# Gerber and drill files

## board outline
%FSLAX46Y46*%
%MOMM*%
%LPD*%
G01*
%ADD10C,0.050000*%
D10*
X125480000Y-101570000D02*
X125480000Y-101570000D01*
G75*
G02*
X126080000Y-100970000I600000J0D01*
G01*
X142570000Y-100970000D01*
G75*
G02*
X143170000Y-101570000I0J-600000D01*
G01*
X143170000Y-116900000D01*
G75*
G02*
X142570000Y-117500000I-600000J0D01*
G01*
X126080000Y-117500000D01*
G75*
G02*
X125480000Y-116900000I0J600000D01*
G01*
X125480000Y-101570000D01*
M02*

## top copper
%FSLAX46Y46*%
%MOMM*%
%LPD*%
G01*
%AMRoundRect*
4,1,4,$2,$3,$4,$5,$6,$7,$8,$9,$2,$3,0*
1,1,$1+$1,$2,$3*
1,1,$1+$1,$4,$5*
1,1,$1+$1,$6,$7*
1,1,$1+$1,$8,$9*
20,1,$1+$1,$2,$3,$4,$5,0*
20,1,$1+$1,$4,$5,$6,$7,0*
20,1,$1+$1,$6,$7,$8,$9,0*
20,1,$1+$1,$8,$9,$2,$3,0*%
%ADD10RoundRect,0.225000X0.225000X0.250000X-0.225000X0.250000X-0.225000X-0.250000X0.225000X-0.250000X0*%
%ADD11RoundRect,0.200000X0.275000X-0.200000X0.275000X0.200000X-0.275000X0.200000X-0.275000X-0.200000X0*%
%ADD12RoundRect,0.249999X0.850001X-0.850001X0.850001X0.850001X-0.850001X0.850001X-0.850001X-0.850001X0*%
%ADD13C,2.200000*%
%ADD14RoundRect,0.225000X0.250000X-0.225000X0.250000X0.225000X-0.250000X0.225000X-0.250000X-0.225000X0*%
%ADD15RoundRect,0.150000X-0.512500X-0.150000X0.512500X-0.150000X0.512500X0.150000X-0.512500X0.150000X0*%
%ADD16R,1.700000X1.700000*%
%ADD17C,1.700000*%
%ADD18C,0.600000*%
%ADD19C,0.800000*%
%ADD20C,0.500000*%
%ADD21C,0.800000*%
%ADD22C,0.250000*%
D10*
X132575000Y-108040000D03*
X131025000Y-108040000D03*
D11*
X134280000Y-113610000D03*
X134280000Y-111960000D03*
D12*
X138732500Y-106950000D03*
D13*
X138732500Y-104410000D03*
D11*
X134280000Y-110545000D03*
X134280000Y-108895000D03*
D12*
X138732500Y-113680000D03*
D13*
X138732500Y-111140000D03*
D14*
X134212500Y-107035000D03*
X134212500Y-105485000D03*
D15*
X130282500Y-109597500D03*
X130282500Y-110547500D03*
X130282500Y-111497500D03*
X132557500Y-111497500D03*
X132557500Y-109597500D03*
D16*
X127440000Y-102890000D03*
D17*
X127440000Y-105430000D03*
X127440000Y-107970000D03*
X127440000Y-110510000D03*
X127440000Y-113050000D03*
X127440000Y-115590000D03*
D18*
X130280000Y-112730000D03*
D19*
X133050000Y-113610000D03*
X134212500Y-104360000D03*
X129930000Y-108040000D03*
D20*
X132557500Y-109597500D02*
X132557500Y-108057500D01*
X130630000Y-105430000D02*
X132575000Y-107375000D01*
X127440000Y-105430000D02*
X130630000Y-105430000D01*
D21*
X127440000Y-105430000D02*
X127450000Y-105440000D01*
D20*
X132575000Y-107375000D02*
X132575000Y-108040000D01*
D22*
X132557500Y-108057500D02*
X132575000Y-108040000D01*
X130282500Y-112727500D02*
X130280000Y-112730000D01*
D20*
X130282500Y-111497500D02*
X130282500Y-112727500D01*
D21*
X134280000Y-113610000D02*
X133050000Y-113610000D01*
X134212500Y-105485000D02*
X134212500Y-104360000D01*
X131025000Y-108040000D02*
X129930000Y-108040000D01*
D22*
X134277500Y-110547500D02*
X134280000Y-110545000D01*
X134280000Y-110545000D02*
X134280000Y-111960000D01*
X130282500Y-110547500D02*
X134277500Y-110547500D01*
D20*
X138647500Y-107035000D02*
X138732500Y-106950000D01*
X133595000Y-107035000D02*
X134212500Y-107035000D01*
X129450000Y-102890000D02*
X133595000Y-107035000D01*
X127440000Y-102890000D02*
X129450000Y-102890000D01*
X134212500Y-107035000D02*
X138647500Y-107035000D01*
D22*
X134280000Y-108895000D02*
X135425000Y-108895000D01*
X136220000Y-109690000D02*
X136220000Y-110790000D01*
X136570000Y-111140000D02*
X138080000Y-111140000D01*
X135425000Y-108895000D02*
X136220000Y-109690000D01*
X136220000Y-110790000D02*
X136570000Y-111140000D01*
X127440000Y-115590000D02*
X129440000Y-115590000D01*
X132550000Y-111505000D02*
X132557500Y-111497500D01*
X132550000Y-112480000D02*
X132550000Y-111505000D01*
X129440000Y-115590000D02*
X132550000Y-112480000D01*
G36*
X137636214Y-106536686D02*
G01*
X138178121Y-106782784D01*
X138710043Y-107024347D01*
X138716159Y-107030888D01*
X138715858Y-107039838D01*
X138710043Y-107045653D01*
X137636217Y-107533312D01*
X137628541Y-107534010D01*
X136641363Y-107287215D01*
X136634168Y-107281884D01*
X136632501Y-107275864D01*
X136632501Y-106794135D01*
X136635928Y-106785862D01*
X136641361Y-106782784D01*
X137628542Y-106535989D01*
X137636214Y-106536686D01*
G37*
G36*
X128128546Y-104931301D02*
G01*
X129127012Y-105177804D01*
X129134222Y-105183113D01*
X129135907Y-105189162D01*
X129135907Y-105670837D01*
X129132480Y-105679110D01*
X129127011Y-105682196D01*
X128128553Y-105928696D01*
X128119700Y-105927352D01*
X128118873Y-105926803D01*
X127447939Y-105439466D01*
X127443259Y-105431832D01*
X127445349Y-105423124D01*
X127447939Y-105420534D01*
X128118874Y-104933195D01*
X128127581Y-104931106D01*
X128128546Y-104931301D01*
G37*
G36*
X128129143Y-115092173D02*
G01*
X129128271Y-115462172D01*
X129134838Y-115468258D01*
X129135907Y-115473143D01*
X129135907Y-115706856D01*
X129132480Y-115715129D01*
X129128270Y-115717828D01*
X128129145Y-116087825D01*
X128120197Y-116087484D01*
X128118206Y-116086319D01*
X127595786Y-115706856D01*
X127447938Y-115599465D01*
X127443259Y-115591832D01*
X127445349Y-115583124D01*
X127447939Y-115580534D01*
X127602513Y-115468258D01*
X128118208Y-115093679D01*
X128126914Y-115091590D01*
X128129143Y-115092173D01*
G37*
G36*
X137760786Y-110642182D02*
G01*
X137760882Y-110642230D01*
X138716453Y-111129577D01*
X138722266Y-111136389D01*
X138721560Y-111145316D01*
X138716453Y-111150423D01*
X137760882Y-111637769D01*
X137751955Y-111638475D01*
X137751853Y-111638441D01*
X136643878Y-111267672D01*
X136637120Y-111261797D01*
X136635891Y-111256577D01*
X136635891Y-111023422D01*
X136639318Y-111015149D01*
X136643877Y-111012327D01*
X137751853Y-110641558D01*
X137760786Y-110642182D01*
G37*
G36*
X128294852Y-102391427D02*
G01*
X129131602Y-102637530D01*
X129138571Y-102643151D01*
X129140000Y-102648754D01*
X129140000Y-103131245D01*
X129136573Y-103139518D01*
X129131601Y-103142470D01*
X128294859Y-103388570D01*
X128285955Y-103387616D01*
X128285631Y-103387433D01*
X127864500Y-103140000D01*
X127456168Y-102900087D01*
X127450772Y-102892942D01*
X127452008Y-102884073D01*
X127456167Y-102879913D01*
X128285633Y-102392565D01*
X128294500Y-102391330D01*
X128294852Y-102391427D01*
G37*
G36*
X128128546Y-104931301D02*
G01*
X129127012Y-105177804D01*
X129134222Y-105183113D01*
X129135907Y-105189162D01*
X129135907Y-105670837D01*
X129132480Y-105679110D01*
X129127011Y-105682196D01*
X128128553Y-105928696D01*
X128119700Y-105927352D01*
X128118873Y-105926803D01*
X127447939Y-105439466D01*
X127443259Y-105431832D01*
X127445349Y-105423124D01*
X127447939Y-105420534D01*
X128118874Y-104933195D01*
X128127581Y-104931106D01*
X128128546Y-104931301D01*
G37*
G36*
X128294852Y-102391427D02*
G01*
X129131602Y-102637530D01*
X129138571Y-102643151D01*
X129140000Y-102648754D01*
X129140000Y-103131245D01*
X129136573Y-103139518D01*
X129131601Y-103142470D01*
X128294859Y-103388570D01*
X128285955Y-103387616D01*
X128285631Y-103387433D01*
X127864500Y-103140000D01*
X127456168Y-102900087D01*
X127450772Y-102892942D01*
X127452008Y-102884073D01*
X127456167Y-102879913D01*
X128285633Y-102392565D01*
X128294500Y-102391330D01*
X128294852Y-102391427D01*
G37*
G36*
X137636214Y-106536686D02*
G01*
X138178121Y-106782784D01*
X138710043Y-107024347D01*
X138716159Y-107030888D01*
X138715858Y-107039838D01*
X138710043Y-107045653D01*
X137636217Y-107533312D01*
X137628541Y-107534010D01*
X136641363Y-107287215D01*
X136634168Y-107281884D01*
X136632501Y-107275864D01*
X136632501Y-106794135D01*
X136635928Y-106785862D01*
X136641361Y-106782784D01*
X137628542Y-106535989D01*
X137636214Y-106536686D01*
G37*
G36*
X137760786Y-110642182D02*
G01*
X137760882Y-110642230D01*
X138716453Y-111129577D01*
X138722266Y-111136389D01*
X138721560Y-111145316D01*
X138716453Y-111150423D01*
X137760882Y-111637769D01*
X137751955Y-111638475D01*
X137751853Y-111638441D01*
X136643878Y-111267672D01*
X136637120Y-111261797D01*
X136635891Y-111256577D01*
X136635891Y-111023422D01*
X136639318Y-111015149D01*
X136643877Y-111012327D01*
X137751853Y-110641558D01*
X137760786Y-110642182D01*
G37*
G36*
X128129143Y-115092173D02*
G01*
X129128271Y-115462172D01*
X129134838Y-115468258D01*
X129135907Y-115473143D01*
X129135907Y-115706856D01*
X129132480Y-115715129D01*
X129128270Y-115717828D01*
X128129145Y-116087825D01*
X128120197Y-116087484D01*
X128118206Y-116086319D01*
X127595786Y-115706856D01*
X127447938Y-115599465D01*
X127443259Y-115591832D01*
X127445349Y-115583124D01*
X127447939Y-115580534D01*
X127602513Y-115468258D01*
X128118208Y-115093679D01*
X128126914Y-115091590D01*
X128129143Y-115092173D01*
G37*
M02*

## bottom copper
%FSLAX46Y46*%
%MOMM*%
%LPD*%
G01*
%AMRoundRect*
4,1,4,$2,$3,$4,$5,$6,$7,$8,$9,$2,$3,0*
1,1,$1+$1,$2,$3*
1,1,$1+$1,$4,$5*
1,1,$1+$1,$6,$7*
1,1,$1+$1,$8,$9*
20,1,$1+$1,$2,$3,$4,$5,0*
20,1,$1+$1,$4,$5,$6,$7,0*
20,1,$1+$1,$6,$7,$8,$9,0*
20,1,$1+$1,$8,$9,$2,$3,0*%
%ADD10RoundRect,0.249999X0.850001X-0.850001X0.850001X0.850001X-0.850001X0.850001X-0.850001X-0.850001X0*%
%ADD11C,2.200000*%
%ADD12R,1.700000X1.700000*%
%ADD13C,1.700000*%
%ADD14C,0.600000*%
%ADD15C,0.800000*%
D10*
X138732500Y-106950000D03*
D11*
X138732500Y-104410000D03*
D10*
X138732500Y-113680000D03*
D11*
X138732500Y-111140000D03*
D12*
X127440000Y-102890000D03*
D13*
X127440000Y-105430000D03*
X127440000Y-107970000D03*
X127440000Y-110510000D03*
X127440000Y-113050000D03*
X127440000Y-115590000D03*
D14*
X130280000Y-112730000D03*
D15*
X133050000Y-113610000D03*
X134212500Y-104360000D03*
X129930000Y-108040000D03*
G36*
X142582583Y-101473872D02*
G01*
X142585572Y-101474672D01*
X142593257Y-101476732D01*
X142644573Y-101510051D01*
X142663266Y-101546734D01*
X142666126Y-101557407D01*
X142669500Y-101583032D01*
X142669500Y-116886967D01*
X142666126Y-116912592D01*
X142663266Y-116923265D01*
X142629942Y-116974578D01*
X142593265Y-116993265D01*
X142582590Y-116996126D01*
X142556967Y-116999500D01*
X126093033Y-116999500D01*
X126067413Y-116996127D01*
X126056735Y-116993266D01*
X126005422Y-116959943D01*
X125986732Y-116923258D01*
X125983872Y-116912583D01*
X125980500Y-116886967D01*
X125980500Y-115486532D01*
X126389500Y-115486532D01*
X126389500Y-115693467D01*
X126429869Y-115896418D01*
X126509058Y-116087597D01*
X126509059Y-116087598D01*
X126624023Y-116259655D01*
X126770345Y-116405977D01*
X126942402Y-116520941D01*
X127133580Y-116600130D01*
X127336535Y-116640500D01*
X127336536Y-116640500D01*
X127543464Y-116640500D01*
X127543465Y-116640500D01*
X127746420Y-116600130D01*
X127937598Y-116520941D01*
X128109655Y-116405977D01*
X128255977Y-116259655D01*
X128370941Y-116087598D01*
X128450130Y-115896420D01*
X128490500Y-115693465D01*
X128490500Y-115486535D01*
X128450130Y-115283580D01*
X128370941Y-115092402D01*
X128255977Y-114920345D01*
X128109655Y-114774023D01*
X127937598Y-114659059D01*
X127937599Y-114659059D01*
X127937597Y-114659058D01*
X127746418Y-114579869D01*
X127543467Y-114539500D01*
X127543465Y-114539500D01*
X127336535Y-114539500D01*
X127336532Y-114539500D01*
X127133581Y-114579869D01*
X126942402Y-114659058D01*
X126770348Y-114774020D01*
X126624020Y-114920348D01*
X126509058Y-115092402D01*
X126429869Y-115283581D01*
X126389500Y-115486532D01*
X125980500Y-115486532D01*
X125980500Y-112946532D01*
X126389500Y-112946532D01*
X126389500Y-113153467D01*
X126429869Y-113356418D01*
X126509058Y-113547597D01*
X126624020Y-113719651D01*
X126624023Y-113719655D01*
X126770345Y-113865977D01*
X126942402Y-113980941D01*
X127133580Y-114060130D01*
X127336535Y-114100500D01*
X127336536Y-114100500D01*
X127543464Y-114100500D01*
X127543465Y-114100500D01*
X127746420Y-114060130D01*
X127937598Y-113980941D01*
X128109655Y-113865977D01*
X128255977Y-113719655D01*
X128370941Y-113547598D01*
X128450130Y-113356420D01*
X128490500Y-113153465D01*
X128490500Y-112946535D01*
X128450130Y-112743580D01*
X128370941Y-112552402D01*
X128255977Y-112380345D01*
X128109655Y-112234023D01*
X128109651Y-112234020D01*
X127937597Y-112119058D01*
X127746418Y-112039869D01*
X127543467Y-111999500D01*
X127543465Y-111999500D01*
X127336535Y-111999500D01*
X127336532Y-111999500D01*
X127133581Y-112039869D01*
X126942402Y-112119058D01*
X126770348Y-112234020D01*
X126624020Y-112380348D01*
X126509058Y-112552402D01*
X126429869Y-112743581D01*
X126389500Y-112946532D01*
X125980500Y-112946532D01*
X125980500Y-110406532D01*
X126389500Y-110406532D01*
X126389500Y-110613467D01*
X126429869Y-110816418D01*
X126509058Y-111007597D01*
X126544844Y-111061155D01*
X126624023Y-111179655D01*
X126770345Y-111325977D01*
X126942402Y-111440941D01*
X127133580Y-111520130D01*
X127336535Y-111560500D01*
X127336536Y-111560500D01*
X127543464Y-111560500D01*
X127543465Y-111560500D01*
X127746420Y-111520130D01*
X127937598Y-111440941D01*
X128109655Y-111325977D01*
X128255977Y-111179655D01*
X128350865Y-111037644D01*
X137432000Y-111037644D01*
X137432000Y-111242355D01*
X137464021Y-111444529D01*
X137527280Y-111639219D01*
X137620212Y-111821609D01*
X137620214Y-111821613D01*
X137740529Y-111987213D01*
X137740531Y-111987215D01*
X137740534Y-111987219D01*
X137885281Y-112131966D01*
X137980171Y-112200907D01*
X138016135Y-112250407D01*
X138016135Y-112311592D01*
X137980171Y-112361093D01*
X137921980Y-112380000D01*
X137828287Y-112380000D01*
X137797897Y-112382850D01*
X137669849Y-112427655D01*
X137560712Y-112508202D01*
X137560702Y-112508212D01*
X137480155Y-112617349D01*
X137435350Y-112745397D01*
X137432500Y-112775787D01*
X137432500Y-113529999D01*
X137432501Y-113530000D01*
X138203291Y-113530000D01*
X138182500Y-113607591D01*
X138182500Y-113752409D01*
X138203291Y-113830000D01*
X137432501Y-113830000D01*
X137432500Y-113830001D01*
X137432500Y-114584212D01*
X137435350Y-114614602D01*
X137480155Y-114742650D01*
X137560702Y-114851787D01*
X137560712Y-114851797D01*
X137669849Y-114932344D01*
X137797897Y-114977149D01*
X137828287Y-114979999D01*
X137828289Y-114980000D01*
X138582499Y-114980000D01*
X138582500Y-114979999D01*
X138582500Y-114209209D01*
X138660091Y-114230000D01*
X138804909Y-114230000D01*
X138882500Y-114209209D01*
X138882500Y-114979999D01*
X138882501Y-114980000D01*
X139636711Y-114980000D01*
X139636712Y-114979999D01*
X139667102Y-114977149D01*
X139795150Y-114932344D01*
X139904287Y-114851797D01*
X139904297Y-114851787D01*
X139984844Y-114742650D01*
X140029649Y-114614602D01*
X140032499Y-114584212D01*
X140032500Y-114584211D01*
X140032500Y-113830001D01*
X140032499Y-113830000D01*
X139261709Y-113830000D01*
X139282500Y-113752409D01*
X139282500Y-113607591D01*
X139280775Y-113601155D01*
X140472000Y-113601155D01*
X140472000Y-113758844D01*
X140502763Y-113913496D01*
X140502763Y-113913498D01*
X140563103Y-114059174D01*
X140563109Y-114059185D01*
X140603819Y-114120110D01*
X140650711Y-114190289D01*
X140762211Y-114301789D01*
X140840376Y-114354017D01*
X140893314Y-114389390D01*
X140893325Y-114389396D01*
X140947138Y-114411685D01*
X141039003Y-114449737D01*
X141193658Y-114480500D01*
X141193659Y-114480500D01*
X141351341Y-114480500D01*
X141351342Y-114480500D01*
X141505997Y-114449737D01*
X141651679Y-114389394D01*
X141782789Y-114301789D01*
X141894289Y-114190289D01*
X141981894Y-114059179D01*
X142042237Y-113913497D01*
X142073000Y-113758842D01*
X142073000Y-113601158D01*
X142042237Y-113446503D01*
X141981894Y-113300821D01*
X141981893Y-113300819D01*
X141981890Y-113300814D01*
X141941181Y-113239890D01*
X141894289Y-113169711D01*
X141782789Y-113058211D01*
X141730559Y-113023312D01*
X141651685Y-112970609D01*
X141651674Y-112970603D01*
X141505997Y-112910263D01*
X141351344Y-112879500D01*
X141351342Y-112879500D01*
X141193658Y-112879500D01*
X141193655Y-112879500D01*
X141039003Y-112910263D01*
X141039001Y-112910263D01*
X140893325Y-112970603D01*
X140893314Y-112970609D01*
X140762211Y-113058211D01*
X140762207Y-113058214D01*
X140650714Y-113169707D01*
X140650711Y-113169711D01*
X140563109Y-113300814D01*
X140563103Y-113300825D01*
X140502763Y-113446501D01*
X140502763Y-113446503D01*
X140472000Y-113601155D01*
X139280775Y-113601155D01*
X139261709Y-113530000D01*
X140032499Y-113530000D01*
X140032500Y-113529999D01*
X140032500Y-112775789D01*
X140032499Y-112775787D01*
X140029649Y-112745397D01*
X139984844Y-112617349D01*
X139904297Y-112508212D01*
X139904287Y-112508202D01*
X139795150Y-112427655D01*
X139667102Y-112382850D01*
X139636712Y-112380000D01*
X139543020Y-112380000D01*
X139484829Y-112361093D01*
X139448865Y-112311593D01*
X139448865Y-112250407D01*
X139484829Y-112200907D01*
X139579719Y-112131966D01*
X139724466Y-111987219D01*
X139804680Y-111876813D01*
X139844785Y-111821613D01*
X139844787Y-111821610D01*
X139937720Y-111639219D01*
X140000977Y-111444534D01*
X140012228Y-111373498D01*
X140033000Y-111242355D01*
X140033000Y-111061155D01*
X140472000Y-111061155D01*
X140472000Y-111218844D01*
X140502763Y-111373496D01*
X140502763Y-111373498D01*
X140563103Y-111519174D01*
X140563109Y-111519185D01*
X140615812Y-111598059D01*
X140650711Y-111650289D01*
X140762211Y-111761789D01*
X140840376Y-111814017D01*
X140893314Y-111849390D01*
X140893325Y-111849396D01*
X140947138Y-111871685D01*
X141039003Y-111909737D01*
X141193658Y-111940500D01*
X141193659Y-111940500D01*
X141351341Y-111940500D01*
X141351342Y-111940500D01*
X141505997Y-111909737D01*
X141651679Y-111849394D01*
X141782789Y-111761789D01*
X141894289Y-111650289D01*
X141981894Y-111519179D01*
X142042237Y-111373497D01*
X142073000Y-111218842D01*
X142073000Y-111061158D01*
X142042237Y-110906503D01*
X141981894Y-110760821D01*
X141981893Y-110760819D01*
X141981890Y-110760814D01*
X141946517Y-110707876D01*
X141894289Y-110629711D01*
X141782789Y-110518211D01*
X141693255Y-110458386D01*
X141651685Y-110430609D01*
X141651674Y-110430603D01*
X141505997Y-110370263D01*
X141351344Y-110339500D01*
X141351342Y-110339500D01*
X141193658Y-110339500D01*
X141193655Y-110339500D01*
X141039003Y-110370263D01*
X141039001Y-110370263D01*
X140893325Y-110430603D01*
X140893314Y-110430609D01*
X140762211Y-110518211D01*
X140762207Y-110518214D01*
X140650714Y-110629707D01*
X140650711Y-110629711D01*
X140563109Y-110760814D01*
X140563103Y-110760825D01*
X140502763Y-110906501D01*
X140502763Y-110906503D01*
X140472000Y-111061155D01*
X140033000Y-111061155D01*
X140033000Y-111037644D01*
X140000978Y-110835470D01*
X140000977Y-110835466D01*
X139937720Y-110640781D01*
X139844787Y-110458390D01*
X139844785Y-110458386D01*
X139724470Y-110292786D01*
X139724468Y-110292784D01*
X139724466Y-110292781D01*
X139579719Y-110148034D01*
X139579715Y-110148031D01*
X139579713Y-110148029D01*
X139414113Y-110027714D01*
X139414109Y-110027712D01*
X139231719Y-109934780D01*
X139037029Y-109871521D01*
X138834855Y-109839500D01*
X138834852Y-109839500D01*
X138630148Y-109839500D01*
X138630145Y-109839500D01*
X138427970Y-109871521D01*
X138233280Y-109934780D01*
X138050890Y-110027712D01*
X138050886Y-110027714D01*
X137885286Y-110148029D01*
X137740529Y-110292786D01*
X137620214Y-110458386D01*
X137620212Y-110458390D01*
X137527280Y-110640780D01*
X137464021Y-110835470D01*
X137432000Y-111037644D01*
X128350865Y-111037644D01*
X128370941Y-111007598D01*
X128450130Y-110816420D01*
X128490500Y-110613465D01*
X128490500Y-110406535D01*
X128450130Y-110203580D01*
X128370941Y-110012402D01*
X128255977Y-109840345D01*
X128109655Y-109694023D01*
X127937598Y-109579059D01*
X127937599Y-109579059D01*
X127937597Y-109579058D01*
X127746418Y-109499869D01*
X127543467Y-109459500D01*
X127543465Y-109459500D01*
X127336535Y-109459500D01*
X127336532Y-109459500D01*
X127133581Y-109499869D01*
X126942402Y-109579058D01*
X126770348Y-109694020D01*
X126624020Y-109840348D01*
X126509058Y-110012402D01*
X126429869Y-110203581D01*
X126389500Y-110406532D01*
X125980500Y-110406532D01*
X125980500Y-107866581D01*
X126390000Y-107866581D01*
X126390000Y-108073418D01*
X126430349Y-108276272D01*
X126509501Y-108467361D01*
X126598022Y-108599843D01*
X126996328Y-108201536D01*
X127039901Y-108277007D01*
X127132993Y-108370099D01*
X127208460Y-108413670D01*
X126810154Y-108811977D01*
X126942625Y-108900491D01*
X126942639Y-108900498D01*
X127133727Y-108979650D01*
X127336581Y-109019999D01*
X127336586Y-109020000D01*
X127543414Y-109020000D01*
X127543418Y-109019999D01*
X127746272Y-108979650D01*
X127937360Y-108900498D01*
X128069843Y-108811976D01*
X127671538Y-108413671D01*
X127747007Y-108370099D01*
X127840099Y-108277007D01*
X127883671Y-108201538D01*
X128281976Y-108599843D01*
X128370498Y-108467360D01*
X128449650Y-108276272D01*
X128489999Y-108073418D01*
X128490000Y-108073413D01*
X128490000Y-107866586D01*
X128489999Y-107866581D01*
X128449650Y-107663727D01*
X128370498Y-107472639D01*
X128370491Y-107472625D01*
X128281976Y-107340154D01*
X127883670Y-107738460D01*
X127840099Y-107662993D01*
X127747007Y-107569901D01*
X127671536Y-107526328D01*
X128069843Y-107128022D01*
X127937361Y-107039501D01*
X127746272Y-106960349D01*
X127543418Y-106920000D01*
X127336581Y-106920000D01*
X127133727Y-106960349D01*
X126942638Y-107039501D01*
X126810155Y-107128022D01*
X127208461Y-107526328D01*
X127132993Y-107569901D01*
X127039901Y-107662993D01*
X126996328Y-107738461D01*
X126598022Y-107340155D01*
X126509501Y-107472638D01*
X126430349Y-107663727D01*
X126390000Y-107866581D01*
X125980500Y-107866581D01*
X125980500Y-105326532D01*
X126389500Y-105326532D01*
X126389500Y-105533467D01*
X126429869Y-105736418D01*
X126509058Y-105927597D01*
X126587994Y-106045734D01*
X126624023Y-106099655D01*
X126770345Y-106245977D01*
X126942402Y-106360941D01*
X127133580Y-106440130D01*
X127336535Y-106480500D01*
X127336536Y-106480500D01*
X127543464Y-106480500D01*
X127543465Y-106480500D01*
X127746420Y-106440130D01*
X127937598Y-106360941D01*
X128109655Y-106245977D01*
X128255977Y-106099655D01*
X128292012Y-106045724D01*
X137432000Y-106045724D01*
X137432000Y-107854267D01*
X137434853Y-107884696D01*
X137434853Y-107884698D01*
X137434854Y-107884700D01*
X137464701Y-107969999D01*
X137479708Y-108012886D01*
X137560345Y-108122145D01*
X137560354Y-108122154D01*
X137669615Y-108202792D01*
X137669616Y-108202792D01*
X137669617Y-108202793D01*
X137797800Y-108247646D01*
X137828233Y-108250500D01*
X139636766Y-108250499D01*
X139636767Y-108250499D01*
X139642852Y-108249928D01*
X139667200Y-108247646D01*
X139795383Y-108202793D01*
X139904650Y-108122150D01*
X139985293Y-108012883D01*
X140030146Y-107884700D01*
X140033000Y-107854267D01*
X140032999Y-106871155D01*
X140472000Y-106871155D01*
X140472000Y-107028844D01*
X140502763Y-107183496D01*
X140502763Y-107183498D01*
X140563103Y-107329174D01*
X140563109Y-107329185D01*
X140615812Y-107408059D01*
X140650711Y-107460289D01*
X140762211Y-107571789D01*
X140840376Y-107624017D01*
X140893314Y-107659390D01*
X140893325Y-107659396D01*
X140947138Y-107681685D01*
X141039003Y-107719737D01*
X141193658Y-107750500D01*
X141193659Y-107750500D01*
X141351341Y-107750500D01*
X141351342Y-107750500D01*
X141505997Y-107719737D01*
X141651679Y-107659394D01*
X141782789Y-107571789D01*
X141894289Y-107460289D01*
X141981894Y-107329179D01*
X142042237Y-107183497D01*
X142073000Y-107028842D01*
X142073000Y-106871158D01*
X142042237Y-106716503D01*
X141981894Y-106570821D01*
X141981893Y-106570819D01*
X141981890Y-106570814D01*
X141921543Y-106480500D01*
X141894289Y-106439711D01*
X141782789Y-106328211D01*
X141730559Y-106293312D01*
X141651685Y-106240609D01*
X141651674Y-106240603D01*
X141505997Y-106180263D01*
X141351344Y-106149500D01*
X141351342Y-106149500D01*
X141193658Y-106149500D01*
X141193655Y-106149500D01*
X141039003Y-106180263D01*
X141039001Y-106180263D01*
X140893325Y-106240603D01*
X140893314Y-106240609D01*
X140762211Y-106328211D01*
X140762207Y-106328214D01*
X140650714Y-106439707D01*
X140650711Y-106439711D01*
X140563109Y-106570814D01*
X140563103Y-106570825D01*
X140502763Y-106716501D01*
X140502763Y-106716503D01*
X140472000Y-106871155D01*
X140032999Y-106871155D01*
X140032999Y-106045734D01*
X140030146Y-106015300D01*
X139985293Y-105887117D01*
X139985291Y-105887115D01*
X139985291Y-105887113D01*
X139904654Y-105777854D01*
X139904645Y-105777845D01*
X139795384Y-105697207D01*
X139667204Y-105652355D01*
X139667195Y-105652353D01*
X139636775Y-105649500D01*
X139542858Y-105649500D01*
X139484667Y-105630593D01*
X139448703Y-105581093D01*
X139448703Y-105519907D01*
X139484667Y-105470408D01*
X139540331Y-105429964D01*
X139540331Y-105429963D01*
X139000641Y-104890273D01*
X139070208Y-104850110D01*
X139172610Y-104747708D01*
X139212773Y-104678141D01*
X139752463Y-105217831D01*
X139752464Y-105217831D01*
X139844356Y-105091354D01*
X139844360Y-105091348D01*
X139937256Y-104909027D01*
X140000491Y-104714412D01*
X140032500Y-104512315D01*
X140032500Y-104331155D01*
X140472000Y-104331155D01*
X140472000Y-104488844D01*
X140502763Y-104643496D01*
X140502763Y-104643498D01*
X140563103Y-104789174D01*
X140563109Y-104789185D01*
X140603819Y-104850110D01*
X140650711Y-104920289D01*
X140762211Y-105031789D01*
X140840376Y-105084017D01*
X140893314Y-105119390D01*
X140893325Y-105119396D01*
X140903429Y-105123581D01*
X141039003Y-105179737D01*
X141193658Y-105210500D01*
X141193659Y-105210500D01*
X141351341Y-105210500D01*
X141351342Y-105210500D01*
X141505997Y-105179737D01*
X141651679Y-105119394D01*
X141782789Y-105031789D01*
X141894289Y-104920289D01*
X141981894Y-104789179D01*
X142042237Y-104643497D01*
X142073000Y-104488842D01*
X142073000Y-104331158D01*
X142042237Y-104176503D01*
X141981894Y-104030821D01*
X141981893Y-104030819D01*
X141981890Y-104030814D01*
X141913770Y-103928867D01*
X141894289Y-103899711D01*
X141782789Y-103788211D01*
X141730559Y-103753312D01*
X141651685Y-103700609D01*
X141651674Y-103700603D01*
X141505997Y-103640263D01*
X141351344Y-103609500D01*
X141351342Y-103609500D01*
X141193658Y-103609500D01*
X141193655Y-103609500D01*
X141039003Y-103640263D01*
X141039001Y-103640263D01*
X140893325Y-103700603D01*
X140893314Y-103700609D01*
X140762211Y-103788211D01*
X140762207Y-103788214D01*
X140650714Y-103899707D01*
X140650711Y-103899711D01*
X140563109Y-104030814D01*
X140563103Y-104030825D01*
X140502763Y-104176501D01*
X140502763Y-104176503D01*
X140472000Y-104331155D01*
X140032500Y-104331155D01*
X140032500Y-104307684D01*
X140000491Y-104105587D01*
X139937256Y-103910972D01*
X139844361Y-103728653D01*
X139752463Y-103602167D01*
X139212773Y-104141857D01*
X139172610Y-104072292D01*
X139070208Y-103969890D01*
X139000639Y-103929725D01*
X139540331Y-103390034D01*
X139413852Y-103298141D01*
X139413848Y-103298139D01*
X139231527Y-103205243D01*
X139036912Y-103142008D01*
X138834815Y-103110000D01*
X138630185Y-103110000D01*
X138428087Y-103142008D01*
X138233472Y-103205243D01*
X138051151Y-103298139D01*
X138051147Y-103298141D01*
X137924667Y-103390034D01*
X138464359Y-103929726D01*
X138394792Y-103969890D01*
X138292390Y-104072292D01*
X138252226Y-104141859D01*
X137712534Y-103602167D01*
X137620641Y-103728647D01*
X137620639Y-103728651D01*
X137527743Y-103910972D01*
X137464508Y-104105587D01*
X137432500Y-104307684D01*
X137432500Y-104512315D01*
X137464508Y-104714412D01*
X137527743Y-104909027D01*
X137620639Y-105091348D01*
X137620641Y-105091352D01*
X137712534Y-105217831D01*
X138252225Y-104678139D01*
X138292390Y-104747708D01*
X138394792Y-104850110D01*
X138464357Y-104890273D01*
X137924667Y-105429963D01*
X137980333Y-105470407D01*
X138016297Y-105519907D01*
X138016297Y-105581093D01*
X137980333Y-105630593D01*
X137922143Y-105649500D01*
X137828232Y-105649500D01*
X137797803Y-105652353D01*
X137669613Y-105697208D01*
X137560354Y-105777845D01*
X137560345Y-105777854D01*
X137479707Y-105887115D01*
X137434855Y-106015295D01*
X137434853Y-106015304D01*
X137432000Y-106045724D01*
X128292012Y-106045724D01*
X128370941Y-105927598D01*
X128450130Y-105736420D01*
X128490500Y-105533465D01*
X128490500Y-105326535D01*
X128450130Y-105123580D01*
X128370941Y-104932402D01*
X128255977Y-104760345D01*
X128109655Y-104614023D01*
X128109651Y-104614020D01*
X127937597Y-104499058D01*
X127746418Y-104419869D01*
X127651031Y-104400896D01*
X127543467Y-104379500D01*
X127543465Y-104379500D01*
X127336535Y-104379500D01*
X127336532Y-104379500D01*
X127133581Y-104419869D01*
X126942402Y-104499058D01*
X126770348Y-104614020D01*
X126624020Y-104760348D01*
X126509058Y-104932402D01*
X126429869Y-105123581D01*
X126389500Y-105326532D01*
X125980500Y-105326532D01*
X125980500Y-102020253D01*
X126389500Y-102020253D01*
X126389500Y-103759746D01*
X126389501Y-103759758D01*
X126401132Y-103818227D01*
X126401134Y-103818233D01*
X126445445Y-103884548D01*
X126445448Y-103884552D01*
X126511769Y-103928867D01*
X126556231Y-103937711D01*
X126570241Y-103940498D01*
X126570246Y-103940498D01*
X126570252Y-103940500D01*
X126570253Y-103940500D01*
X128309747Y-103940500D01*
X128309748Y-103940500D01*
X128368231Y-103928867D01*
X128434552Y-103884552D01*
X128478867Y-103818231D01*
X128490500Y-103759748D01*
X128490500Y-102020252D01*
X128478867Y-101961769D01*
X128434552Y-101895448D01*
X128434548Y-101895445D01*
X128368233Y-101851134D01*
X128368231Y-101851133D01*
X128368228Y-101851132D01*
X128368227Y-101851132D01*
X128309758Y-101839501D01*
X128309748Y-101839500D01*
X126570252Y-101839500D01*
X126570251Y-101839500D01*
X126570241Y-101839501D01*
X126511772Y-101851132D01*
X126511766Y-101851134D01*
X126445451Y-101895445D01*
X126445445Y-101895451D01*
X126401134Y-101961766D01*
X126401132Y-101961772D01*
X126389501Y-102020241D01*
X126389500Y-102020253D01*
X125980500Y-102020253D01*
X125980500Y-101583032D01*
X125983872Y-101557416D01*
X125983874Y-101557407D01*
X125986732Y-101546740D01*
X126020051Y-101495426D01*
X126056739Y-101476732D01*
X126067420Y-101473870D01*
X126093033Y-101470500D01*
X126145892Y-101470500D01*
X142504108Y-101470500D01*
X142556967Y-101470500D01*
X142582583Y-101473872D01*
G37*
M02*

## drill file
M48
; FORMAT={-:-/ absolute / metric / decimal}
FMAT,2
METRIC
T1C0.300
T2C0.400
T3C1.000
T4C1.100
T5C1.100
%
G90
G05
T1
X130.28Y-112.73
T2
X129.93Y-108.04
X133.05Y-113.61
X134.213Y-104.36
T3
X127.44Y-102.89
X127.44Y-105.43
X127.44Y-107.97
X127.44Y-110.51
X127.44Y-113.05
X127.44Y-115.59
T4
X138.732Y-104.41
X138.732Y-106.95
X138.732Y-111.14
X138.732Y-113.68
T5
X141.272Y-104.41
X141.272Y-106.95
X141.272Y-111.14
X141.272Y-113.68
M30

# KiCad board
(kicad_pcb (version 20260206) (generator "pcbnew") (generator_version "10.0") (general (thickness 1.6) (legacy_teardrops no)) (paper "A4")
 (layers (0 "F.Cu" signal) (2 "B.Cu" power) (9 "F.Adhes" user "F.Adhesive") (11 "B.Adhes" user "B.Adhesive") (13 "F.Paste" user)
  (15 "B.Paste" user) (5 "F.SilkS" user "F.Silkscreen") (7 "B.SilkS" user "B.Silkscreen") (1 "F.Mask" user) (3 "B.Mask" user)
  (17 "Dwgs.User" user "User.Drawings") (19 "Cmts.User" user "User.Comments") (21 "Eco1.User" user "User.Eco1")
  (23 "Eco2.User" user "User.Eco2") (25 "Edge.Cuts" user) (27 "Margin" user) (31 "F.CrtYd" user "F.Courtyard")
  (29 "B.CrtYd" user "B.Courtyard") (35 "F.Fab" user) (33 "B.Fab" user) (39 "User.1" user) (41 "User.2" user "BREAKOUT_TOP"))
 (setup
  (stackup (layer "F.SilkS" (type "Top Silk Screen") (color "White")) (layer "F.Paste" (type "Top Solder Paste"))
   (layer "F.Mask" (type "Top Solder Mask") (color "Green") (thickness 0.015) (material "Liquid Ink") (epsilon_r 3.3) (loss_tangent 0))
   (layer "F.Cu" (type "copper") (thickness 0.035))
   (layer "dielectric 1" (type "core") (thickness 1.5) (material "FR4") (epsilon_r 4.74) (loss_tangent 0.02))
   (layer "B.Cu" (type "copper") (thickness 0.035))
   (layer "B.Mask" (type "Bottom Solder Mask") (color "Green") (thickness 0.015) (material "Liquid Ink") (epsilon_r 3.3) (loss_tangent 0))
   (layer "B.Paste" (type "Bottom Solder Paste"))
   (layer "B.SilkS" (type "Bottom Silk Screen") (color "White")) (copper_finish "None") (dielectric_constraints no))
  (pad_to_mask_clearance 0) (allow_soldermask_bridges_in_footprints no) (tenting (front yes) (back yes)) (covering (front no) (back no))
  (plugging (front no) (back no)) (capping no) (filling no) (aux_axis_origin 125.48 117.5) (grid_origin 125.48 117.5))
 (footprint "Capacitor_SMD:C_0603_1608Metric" (layer "F.Cu") (at 131.8 108.04 180)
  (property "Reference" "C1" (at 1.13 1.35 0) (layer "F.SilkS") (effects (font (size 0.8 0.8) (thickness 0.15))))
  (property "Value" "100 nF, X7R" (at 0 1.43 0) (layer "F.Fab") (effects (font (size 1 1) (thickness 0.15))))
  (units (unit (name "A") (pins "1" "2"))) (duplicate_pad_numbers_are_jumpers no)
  (pad "1" smd roundrect (at -0.775 0 180) (size 0.9 0.95) (layers "F.Cu" "F.Mask" "F.Paste") (roundrect_rratio 0.25) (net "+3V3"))
  (pad "2" smd roundrect (at 0.775 0 180) (size 0.9 0.95) (layers "F.Cu" "F.Mask" "F.Paste") (roundrect_rratio 0.25) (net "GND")))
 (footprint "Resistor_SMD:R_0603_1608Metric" (layer "F.Cu") (at 134.28 112.785 90)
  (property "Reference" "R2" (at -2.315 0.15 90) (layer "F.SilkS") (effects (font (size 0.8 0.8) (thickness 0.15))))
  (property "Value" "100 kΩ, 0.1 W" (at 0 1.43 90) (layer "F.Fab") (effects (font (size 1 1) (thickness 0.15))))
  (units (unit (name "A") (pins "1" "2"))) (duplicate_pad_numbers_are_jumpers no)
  (pad "1" smd roundrect (at -0.825 0 90) (size 0.8 0.95) (layers "F.Cu" "F.Mask" "F.Paste") (roundrect_rratio 0.25) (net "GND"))
  (pad "2" smd roundrect (at 0.825 0 90) (size 0.8 0.95) (layers "F.Cu" "F.Mask" "F.Paste") (roundrect_rratio 0.25) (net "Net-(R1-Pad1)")))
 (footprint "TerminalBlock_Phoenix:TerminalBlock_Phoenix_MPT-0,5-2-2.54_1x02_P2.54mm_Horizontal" (layer "F.Cu") (at 138.7325 106.95 90)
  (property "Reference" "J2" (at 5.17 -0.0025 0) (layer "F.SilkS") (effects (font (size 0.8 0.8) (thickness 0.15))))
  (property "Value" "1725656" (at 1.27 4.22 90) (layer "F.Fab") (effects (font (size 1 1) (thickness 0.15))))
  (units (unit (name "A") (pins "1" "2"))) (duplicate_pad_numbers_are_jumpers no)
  (pad "" np_thru_hole circle (at 0 2.54 90) (size 1.1 1.1) (drill 1.1) (layers "*.Cu" "*.Mask"))
  (pad "" np_thru_hole circle (at 2.54 2.54 90) (size 1.1 1.1) (drill 1.1) (layers "*.Cu" "*.Mask"))
  (pad "1" thru_hole roundrect (at 0 0 90) (size 2.2 2.2) (drill 1.1) (layers "*.Cu" "*.Mask") (remove_unused_layers no)
   (roundrect_rratio 0.113636) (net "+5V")
   (teardrops (best_length_ratio 0.5) (max_length 1) (best_width_ratio 1) (max_width 1) (curved_edges no) (filter_ratio 0.9) (enabled yes)
    (allow_two_segments no) (prefer_zone_connections yes)))
  (pad "2" thru_hole circle (at 2.54 0 90) (size 2.2 2.2) (drill 1.1) (layers "*.Cu" "*.Mask") (remove_unused_layers no) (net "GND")
   (teardrops (best_length_ratio 0.5) (max_length 1) (best_width_ratio 1) (max_width 1) (curved_edges no) (filter_ratio 0.9) (enabled yes)
    (allow_two_segments no) (prefer_zone_connections yes))))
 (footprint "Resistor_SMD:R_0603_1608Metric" (layer "F.Cu") (at 134.28 109.72 90)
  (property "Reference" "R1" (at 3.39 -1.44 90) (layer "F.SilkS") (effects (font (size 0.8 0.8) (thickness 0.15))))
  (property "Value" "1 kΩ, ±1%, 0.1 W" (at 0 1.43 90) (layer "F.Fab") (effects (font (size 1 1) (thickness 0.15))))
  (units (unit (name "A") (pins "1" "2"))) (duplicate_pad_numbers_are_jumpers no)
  (pad "1" smd roundrect (at -0.825 0 90) (size 0.8 0.95) (layers "F.Cu" "F.Mask" "F.Paste") (roundrect_rratio 0.25) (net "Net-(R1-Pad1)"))
  (pad "2" smd roundrect (at 0.825 0 90) (size 0.8 0.95) (layers "F.Cu" "F.Mask" "F.Paste") (roundrect_rratio 0.25) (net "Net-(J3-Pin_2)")))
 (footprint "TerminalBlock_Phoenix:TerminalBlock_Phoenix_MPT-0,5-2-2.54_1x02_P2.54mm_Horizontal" (layer "F.Cu") (at 138.7325 113.68 90)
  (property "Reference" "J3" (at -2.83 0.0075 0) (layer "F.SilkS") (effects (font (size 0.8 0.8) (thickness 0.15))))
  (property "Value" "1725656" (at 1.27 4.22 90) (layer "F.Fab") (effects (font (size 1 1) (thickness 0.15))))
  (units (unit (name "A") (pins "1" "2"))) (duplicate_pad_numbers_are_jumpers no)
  (pad "" np_thru_hole circle (at 0 2.54 90) (size 1.1 1.1) (drill 1.1) (layers "*.Cu" "*.Mask"))
  (pad "" np_thru_hole circle (at 2.54 2.54 90) (size 1.1 1.1) (drill 1.1) (layers "*.Cu" "*.Mask"))
  (pad "1" thru_hole roundrect (at 0 0 90) (size 2.2 2.2) (drill 1.1) (layers "*.Cu" "*.Mask") (remove_unused_layers no)
   (roundrect_rratio 0.113636) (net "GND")
   (teardrops (best_length_ratio 0.5) (max_length 1) (best_width_ratio 1) (max_width 1) (curved_edges no) (filter_ratio 0.9) (enabled yes)
    (allow_two_segments no) (prefer_zone_connections yes)))
  (pad "2" thru_hole circle (at 2.54 0 90) (size 2.2 2.2) (drill 1.1) (layers "*.Cu" "*.Mask") (remove_unused_layers no)
   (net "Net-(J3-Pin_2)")
   (teardrops (best_length_ratio 0.5) (max_length 1) (best_width_ratio 1) (max_width 1) (curved_edges no) (filter_ratio 0.9) (enabled yes)
    (allow_two_segments no) (prefer_zone_connections yes))))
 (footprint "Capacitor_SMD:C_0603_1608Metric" (layer "F.Cu") (at 134.2125 106.26 90)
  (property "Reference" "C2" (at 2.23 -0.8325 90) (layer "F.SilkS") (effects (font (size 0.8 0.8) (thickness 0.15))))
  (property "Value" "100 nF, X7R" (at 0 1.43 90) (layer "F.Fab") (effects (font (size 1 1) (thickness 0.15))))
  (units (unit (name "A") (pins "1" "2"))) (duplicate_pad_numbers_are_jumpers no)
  (pad "1" smd roundrect (at -0.775 0 90) (size 0.9 0.95) (layers "F.Cu" "F.Mask" "F.Paste") (roundrect_rratio 0.25) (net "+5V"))
  (pad "2" smd roundrect (at 0.775 0 90) (size 0.9 0.95) (layers "F.Cu" "F.Mask" "F.Paste") (roundrect_rratio 0.25) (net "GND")))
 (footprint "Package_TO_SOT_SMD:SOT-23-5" (layer "F.Cu") (at 131.42 110.5475)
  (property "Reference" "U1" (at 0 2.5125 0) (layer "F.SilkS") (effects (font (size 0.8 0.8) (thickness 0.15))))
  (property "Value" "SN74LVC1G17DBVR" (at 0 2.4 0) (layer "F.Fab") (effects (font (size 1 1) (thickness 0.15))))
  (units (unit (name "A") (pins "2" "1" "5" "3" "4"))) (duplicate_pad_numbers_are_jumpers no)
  (pad "1" smd roundrect (at -1.1375 -0.95) (size 1.325 0.6) (layers "F.Cu" "F.Mask" "F.Paste") (roundrect_rratio 0.25)
   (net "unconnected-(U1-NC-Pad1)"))
  (pad "2" smd roundrect (at -1.1375 0) (size 1.325 0.6) (layers "F.Cu" "F.Mask" "F.Paste") (roundrect_rratio 0.25) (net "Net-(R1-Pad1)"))
  (pad "3" smd roundrect (at -1.1375 0.95) (size 1.325 0.6) (layers "F.Cu" "F.Mask" "F.Paste") (roundrect_rratio 0.25) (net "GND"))
  (pad "4" smd roundrect (at 1.1375 0.95) (size 1.325 0.6) (layers "F.Cu" "F.Mask" "F.Paste") (roundrect_rratio 0.25) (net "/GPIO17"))
  (pad "5" smd roundrect (at 1.1375 -0.95) (size 1.325 0.6) (layers "F.Cu" "F.Mask" "F.Paste") (roundrect_rratio 0.25) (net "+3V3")))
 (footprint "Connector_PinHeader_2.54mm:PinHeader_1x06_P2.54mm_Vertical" (layer "B.Cu") (at 127.44 102.89 180)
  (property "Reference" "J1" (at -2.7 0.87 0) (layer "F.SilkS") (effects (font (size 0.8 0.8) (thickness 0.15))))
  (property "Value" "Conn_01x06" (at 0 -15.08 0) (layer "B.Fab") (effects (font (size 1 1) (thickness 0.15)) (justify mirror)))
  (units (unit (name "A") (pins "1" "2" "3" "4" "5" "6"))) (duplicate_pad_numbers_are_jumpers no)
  (pad "1" thru_hole rect (at 0 0 180) (size 1.7 1.7) (drill 1) (layers "*.Cu" "*.Mask") (remove_unused_layers no) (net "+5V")
   (teardrops (best_length_ratio 0.5) (max_length 1) (best_width_ratio 1) (max_width 1) (curved_edges no) (filter_ratio 0.9) (enabled yes)
    (allow_two_segments no) (prefer_zone_connections yes)))
  (pad "2" thru_hole circle (at 0 -2.54 180) (size 1.7 1.7) (drill 1) (layers "*.Cu" "*.Mask") (remove_unused_layers no) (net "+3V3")
   (teardrops (best_length_ratio 0.5) (max_length 1) (best_width_ratio 1) (max_width 1) (curved_edges no) (filter_ratio 0.9) (enabled yes)
    (allow_two_segments no) (prefer_zone_connections yes)))
  (pad "3" thru_hole circle (at 0 -5.08 180) (size 1.7 1.7) (drill 1) (layers "*.Cu" "*.Mask") (remove_unused_layers no) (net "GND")
   (teardrops (best_length_ratio 0.5) (max_length 1) (best_width_ratio 1) (max_width 1) (curved_edges no) (filter_ratio 0.9) (enabled yes)
    (allow_two_segments no) (prefer_zone_connections yes)))
  (pad "4" thru_hole circle (at 0 -7.62 180) (size 1.7 1.7) (drill 1) (layers "*.Cu" "*.Mask") (remove_unused_layers no)
   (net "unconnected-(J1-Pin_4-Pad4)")
   (teardrops (best_length_ratio 0.5) (max_length 1) (best_width_ratio 1) (max_width 1) (curved_edges no) (filter_ratio 0.9) (enabled yes)
    (allow_two_segments no) (prefer_zone_connections yes)))
  (pad "5" thru_hole circle (at 0 -10.16 180) (size 1.7 1.7) (drill 1) (layers "*.Cu" "*.Mask") (remove_unused_layers no)
   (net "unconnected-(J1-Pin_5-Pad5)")
   (teardrops (best_length_ratio 0.5) (max_length 1) (best_width_ratio 1) (max_width 1) (curved_edges no) (filter_ratio 0.9) (enabled yes)
    (allow_two_segments no) (prefer_zone_connections yes)))
  (pad "6" thru_hole circle (at 0 -12.7 180) (size 1.7 1.7) (drill 1) (layers "*.Cu" "*.Mask") (remove_unused_layers no) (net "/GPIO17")
   (teardrops (best_length_ratio 0.5) (max_length 1) (best_width_ratio 1) (max_width 1) (curved_edges no) (filter_ratio 0.9) (enabled yes)
    (allow_two_segments no) (prefer_zone_connections yes))))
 (gr_rect (start 125.48 100.97) (end 143.17 117.5) (radius 0.6) (stroke (width 0.05) (type solid)) (fill no) (layer "Edge.Cuts"))
 (segment (start 132.5575 109.5975) (end 132.5575 108.0575) (width 0.5) (layer "F.Cu") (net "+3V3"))
 (segment (start 130.63 105.43) (end 132.575 107.375) (width 0.5) (layer "F.Cu") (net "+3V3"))
 (segment (start 127.44 105.43) (end 130.63 105.43) (width 0.5) (layer "F.Cu") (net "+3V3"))
 (segment (start 127.44 105.43) (end 127.45 105.44) (width 0.8) (layer "F.Cu") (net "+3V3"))
 (segment (start 132.575 107.375) (end 132.575 108.04) (width 0.5) (layer "F.Cu") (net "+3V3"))
 (segment (start 132.5575 108.0575) (end 132.575 108.04) (width 0.25) (layer "F.Cu") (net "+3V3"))
 (segment (start 130.2825 112.7275) (end 130.28 112.73) (width 0.25) (layer "F.Cu") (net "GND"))
 (segment (start 130.2825 111.4975) (end 130.2825 112.7275) (width 0.5) (layer "F.Cu") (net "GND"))
 (segment (start 134.28 113.61) (end 133.05 113.61) (width 0.8) (layer "F.Cu") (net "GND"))
 (segment (start 134.2125 105.485) (end 134.2125 104.36) (width 0.8) (layer "F.Cu") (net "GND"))
 (segment (start 131.025 108.04) (end 129.93 108.04) (width 0.8) (layer "F.Cu") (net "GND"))
 (via (at 130.28 112.73) (size 0.6) (drill 0.3) (layers "F.Cu" "B.Cu") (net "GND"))
 (via (at 133.05 113.61) (size 0.8) (drill 0.4) (layers "F.Cu" "B.Cu") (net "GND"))
 (via (at 134.2125 104.36) (size 0.8) (drill 0.4) (layers "F.Cu" "B.Cu") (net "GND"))
 (via (at 129.93 108.04) (size 0.8) (drill 0.4) (layers "F.Cu" "B.Cu") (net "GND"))
 (segment (start 134.2775 110.5475) (end 134.28 110.545) (width 0.25) (layer "F.Cu") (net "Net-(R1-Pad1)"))
 (segment (start 134.28 110.545) (end 134.28 111.96) (width 0.25) (layer "F.Cu") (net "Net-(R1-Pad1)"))
 (segment (start 130.2825 110.5475) (end 134.2775 110.5475) (width 0.25) (layer "F.Cu") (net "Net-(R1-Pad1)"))
 (segment (start 138.6475 107.035) (end 138.7325 106.95) (width 0.5) (layer "F.Cu") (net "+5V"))
 (segment (start 133.595 107.035) (end 134.2125 107.035) (width 0.5) (layer "F.Cu") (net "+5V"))
 (segment (start 129.45 102.89) (end 133.595 107.035) (width 0.5) (layer "F.Cu") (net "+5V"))
 (segment (start 127.44 102.89) (end 129.45 102.89) (width 0.5) (layer "F.Cu") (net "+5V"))
 (segment (start 134.2125 107.035) (end 138.6475 107.035) (width 0.5) (layer "F.Cu") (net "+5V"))
 (segment (start 134.28 108.895) (end 135.425 108.895) (width 0.25) (layer "F.Cu") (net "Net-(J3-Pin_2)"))
 (segment (start 136.22 109.69) (end 136.22 110.79) (width 0.25) (layer "F.Cu") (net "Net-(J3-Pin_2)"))
 (segment (start 136.57 111.14) (end 138.08 111.14) (width 0.25) (layer "F.Cu") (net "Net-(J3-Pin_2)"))
 (segment (start 135.425 108.895) (end 136.22 109.69) (width 0.25) (layer "F.Cu") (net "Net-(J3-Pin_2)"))
 (segment (start 136.22 110.79) (end 136.57 111.14) (width 0.25) (layer "F.Cu") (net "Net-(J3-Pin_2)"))
 (segment (start 127.44 115.59) (end 129.44 115.59) (width 0.25) (layer "F.Cu") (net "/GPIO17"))
 (segment (start 132.55 111.505) (end 132.5575 111.4975) (width 0.25) (layer "F.Cu") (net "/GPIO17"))
 (segment (start 132.55 112.48) (end 132.55 111.505) (width 0.25) (layer "F.Cu") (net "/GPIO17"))
 (segment (start 129.44 115.59) (end 132.55 112.48) (width 0.25) (layer "F.Cu") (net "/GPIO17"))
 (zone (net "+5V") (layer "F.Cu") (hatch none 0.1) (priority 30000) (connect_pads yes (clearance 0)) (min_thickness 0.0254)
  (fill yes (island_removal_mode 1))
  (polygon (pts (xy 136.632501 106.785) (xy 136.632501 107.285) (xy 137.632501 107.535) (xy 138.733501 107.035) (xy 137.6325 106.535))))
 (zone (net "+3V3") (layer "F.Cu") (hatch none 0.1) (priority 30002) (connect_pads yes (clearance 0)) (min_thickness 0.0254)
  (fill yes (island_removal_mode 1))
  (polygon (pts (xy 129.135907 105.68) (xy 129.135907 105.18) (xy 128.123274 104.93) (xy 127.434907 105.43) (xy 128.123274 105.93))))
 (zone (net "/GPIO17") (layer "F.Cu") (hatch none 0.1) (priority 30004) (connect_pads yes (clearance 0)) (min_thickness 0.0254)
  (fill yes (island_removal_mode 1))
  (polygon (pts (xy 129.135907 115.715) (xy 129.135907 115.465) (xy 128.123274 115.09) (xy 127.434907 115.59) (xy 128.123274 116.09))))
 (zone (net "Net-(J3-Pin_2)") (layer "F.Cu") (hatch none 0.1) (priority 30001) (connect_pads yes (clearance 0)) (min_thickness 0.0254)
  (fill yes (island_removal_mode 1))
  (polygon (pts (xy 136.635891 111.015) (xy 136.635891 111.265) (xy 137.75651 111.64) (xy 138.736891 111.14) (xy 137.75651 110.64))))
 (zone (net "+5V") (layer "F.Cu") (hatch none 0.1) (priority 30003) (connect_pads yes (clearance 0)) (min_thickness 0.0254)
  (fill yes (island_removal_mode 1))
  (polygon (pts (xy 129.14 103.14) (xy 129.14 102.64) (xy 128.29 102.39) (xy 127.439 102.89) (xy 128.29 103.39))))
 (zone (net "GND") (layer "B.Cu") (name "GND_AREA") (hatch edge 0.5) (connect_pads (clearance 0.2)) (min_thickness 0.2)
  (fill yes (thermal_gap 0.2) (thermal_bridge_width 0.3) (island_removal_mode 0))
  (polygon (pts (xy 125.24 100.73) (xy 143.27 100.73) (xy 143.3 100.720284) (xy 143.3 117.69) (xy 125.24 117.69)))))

